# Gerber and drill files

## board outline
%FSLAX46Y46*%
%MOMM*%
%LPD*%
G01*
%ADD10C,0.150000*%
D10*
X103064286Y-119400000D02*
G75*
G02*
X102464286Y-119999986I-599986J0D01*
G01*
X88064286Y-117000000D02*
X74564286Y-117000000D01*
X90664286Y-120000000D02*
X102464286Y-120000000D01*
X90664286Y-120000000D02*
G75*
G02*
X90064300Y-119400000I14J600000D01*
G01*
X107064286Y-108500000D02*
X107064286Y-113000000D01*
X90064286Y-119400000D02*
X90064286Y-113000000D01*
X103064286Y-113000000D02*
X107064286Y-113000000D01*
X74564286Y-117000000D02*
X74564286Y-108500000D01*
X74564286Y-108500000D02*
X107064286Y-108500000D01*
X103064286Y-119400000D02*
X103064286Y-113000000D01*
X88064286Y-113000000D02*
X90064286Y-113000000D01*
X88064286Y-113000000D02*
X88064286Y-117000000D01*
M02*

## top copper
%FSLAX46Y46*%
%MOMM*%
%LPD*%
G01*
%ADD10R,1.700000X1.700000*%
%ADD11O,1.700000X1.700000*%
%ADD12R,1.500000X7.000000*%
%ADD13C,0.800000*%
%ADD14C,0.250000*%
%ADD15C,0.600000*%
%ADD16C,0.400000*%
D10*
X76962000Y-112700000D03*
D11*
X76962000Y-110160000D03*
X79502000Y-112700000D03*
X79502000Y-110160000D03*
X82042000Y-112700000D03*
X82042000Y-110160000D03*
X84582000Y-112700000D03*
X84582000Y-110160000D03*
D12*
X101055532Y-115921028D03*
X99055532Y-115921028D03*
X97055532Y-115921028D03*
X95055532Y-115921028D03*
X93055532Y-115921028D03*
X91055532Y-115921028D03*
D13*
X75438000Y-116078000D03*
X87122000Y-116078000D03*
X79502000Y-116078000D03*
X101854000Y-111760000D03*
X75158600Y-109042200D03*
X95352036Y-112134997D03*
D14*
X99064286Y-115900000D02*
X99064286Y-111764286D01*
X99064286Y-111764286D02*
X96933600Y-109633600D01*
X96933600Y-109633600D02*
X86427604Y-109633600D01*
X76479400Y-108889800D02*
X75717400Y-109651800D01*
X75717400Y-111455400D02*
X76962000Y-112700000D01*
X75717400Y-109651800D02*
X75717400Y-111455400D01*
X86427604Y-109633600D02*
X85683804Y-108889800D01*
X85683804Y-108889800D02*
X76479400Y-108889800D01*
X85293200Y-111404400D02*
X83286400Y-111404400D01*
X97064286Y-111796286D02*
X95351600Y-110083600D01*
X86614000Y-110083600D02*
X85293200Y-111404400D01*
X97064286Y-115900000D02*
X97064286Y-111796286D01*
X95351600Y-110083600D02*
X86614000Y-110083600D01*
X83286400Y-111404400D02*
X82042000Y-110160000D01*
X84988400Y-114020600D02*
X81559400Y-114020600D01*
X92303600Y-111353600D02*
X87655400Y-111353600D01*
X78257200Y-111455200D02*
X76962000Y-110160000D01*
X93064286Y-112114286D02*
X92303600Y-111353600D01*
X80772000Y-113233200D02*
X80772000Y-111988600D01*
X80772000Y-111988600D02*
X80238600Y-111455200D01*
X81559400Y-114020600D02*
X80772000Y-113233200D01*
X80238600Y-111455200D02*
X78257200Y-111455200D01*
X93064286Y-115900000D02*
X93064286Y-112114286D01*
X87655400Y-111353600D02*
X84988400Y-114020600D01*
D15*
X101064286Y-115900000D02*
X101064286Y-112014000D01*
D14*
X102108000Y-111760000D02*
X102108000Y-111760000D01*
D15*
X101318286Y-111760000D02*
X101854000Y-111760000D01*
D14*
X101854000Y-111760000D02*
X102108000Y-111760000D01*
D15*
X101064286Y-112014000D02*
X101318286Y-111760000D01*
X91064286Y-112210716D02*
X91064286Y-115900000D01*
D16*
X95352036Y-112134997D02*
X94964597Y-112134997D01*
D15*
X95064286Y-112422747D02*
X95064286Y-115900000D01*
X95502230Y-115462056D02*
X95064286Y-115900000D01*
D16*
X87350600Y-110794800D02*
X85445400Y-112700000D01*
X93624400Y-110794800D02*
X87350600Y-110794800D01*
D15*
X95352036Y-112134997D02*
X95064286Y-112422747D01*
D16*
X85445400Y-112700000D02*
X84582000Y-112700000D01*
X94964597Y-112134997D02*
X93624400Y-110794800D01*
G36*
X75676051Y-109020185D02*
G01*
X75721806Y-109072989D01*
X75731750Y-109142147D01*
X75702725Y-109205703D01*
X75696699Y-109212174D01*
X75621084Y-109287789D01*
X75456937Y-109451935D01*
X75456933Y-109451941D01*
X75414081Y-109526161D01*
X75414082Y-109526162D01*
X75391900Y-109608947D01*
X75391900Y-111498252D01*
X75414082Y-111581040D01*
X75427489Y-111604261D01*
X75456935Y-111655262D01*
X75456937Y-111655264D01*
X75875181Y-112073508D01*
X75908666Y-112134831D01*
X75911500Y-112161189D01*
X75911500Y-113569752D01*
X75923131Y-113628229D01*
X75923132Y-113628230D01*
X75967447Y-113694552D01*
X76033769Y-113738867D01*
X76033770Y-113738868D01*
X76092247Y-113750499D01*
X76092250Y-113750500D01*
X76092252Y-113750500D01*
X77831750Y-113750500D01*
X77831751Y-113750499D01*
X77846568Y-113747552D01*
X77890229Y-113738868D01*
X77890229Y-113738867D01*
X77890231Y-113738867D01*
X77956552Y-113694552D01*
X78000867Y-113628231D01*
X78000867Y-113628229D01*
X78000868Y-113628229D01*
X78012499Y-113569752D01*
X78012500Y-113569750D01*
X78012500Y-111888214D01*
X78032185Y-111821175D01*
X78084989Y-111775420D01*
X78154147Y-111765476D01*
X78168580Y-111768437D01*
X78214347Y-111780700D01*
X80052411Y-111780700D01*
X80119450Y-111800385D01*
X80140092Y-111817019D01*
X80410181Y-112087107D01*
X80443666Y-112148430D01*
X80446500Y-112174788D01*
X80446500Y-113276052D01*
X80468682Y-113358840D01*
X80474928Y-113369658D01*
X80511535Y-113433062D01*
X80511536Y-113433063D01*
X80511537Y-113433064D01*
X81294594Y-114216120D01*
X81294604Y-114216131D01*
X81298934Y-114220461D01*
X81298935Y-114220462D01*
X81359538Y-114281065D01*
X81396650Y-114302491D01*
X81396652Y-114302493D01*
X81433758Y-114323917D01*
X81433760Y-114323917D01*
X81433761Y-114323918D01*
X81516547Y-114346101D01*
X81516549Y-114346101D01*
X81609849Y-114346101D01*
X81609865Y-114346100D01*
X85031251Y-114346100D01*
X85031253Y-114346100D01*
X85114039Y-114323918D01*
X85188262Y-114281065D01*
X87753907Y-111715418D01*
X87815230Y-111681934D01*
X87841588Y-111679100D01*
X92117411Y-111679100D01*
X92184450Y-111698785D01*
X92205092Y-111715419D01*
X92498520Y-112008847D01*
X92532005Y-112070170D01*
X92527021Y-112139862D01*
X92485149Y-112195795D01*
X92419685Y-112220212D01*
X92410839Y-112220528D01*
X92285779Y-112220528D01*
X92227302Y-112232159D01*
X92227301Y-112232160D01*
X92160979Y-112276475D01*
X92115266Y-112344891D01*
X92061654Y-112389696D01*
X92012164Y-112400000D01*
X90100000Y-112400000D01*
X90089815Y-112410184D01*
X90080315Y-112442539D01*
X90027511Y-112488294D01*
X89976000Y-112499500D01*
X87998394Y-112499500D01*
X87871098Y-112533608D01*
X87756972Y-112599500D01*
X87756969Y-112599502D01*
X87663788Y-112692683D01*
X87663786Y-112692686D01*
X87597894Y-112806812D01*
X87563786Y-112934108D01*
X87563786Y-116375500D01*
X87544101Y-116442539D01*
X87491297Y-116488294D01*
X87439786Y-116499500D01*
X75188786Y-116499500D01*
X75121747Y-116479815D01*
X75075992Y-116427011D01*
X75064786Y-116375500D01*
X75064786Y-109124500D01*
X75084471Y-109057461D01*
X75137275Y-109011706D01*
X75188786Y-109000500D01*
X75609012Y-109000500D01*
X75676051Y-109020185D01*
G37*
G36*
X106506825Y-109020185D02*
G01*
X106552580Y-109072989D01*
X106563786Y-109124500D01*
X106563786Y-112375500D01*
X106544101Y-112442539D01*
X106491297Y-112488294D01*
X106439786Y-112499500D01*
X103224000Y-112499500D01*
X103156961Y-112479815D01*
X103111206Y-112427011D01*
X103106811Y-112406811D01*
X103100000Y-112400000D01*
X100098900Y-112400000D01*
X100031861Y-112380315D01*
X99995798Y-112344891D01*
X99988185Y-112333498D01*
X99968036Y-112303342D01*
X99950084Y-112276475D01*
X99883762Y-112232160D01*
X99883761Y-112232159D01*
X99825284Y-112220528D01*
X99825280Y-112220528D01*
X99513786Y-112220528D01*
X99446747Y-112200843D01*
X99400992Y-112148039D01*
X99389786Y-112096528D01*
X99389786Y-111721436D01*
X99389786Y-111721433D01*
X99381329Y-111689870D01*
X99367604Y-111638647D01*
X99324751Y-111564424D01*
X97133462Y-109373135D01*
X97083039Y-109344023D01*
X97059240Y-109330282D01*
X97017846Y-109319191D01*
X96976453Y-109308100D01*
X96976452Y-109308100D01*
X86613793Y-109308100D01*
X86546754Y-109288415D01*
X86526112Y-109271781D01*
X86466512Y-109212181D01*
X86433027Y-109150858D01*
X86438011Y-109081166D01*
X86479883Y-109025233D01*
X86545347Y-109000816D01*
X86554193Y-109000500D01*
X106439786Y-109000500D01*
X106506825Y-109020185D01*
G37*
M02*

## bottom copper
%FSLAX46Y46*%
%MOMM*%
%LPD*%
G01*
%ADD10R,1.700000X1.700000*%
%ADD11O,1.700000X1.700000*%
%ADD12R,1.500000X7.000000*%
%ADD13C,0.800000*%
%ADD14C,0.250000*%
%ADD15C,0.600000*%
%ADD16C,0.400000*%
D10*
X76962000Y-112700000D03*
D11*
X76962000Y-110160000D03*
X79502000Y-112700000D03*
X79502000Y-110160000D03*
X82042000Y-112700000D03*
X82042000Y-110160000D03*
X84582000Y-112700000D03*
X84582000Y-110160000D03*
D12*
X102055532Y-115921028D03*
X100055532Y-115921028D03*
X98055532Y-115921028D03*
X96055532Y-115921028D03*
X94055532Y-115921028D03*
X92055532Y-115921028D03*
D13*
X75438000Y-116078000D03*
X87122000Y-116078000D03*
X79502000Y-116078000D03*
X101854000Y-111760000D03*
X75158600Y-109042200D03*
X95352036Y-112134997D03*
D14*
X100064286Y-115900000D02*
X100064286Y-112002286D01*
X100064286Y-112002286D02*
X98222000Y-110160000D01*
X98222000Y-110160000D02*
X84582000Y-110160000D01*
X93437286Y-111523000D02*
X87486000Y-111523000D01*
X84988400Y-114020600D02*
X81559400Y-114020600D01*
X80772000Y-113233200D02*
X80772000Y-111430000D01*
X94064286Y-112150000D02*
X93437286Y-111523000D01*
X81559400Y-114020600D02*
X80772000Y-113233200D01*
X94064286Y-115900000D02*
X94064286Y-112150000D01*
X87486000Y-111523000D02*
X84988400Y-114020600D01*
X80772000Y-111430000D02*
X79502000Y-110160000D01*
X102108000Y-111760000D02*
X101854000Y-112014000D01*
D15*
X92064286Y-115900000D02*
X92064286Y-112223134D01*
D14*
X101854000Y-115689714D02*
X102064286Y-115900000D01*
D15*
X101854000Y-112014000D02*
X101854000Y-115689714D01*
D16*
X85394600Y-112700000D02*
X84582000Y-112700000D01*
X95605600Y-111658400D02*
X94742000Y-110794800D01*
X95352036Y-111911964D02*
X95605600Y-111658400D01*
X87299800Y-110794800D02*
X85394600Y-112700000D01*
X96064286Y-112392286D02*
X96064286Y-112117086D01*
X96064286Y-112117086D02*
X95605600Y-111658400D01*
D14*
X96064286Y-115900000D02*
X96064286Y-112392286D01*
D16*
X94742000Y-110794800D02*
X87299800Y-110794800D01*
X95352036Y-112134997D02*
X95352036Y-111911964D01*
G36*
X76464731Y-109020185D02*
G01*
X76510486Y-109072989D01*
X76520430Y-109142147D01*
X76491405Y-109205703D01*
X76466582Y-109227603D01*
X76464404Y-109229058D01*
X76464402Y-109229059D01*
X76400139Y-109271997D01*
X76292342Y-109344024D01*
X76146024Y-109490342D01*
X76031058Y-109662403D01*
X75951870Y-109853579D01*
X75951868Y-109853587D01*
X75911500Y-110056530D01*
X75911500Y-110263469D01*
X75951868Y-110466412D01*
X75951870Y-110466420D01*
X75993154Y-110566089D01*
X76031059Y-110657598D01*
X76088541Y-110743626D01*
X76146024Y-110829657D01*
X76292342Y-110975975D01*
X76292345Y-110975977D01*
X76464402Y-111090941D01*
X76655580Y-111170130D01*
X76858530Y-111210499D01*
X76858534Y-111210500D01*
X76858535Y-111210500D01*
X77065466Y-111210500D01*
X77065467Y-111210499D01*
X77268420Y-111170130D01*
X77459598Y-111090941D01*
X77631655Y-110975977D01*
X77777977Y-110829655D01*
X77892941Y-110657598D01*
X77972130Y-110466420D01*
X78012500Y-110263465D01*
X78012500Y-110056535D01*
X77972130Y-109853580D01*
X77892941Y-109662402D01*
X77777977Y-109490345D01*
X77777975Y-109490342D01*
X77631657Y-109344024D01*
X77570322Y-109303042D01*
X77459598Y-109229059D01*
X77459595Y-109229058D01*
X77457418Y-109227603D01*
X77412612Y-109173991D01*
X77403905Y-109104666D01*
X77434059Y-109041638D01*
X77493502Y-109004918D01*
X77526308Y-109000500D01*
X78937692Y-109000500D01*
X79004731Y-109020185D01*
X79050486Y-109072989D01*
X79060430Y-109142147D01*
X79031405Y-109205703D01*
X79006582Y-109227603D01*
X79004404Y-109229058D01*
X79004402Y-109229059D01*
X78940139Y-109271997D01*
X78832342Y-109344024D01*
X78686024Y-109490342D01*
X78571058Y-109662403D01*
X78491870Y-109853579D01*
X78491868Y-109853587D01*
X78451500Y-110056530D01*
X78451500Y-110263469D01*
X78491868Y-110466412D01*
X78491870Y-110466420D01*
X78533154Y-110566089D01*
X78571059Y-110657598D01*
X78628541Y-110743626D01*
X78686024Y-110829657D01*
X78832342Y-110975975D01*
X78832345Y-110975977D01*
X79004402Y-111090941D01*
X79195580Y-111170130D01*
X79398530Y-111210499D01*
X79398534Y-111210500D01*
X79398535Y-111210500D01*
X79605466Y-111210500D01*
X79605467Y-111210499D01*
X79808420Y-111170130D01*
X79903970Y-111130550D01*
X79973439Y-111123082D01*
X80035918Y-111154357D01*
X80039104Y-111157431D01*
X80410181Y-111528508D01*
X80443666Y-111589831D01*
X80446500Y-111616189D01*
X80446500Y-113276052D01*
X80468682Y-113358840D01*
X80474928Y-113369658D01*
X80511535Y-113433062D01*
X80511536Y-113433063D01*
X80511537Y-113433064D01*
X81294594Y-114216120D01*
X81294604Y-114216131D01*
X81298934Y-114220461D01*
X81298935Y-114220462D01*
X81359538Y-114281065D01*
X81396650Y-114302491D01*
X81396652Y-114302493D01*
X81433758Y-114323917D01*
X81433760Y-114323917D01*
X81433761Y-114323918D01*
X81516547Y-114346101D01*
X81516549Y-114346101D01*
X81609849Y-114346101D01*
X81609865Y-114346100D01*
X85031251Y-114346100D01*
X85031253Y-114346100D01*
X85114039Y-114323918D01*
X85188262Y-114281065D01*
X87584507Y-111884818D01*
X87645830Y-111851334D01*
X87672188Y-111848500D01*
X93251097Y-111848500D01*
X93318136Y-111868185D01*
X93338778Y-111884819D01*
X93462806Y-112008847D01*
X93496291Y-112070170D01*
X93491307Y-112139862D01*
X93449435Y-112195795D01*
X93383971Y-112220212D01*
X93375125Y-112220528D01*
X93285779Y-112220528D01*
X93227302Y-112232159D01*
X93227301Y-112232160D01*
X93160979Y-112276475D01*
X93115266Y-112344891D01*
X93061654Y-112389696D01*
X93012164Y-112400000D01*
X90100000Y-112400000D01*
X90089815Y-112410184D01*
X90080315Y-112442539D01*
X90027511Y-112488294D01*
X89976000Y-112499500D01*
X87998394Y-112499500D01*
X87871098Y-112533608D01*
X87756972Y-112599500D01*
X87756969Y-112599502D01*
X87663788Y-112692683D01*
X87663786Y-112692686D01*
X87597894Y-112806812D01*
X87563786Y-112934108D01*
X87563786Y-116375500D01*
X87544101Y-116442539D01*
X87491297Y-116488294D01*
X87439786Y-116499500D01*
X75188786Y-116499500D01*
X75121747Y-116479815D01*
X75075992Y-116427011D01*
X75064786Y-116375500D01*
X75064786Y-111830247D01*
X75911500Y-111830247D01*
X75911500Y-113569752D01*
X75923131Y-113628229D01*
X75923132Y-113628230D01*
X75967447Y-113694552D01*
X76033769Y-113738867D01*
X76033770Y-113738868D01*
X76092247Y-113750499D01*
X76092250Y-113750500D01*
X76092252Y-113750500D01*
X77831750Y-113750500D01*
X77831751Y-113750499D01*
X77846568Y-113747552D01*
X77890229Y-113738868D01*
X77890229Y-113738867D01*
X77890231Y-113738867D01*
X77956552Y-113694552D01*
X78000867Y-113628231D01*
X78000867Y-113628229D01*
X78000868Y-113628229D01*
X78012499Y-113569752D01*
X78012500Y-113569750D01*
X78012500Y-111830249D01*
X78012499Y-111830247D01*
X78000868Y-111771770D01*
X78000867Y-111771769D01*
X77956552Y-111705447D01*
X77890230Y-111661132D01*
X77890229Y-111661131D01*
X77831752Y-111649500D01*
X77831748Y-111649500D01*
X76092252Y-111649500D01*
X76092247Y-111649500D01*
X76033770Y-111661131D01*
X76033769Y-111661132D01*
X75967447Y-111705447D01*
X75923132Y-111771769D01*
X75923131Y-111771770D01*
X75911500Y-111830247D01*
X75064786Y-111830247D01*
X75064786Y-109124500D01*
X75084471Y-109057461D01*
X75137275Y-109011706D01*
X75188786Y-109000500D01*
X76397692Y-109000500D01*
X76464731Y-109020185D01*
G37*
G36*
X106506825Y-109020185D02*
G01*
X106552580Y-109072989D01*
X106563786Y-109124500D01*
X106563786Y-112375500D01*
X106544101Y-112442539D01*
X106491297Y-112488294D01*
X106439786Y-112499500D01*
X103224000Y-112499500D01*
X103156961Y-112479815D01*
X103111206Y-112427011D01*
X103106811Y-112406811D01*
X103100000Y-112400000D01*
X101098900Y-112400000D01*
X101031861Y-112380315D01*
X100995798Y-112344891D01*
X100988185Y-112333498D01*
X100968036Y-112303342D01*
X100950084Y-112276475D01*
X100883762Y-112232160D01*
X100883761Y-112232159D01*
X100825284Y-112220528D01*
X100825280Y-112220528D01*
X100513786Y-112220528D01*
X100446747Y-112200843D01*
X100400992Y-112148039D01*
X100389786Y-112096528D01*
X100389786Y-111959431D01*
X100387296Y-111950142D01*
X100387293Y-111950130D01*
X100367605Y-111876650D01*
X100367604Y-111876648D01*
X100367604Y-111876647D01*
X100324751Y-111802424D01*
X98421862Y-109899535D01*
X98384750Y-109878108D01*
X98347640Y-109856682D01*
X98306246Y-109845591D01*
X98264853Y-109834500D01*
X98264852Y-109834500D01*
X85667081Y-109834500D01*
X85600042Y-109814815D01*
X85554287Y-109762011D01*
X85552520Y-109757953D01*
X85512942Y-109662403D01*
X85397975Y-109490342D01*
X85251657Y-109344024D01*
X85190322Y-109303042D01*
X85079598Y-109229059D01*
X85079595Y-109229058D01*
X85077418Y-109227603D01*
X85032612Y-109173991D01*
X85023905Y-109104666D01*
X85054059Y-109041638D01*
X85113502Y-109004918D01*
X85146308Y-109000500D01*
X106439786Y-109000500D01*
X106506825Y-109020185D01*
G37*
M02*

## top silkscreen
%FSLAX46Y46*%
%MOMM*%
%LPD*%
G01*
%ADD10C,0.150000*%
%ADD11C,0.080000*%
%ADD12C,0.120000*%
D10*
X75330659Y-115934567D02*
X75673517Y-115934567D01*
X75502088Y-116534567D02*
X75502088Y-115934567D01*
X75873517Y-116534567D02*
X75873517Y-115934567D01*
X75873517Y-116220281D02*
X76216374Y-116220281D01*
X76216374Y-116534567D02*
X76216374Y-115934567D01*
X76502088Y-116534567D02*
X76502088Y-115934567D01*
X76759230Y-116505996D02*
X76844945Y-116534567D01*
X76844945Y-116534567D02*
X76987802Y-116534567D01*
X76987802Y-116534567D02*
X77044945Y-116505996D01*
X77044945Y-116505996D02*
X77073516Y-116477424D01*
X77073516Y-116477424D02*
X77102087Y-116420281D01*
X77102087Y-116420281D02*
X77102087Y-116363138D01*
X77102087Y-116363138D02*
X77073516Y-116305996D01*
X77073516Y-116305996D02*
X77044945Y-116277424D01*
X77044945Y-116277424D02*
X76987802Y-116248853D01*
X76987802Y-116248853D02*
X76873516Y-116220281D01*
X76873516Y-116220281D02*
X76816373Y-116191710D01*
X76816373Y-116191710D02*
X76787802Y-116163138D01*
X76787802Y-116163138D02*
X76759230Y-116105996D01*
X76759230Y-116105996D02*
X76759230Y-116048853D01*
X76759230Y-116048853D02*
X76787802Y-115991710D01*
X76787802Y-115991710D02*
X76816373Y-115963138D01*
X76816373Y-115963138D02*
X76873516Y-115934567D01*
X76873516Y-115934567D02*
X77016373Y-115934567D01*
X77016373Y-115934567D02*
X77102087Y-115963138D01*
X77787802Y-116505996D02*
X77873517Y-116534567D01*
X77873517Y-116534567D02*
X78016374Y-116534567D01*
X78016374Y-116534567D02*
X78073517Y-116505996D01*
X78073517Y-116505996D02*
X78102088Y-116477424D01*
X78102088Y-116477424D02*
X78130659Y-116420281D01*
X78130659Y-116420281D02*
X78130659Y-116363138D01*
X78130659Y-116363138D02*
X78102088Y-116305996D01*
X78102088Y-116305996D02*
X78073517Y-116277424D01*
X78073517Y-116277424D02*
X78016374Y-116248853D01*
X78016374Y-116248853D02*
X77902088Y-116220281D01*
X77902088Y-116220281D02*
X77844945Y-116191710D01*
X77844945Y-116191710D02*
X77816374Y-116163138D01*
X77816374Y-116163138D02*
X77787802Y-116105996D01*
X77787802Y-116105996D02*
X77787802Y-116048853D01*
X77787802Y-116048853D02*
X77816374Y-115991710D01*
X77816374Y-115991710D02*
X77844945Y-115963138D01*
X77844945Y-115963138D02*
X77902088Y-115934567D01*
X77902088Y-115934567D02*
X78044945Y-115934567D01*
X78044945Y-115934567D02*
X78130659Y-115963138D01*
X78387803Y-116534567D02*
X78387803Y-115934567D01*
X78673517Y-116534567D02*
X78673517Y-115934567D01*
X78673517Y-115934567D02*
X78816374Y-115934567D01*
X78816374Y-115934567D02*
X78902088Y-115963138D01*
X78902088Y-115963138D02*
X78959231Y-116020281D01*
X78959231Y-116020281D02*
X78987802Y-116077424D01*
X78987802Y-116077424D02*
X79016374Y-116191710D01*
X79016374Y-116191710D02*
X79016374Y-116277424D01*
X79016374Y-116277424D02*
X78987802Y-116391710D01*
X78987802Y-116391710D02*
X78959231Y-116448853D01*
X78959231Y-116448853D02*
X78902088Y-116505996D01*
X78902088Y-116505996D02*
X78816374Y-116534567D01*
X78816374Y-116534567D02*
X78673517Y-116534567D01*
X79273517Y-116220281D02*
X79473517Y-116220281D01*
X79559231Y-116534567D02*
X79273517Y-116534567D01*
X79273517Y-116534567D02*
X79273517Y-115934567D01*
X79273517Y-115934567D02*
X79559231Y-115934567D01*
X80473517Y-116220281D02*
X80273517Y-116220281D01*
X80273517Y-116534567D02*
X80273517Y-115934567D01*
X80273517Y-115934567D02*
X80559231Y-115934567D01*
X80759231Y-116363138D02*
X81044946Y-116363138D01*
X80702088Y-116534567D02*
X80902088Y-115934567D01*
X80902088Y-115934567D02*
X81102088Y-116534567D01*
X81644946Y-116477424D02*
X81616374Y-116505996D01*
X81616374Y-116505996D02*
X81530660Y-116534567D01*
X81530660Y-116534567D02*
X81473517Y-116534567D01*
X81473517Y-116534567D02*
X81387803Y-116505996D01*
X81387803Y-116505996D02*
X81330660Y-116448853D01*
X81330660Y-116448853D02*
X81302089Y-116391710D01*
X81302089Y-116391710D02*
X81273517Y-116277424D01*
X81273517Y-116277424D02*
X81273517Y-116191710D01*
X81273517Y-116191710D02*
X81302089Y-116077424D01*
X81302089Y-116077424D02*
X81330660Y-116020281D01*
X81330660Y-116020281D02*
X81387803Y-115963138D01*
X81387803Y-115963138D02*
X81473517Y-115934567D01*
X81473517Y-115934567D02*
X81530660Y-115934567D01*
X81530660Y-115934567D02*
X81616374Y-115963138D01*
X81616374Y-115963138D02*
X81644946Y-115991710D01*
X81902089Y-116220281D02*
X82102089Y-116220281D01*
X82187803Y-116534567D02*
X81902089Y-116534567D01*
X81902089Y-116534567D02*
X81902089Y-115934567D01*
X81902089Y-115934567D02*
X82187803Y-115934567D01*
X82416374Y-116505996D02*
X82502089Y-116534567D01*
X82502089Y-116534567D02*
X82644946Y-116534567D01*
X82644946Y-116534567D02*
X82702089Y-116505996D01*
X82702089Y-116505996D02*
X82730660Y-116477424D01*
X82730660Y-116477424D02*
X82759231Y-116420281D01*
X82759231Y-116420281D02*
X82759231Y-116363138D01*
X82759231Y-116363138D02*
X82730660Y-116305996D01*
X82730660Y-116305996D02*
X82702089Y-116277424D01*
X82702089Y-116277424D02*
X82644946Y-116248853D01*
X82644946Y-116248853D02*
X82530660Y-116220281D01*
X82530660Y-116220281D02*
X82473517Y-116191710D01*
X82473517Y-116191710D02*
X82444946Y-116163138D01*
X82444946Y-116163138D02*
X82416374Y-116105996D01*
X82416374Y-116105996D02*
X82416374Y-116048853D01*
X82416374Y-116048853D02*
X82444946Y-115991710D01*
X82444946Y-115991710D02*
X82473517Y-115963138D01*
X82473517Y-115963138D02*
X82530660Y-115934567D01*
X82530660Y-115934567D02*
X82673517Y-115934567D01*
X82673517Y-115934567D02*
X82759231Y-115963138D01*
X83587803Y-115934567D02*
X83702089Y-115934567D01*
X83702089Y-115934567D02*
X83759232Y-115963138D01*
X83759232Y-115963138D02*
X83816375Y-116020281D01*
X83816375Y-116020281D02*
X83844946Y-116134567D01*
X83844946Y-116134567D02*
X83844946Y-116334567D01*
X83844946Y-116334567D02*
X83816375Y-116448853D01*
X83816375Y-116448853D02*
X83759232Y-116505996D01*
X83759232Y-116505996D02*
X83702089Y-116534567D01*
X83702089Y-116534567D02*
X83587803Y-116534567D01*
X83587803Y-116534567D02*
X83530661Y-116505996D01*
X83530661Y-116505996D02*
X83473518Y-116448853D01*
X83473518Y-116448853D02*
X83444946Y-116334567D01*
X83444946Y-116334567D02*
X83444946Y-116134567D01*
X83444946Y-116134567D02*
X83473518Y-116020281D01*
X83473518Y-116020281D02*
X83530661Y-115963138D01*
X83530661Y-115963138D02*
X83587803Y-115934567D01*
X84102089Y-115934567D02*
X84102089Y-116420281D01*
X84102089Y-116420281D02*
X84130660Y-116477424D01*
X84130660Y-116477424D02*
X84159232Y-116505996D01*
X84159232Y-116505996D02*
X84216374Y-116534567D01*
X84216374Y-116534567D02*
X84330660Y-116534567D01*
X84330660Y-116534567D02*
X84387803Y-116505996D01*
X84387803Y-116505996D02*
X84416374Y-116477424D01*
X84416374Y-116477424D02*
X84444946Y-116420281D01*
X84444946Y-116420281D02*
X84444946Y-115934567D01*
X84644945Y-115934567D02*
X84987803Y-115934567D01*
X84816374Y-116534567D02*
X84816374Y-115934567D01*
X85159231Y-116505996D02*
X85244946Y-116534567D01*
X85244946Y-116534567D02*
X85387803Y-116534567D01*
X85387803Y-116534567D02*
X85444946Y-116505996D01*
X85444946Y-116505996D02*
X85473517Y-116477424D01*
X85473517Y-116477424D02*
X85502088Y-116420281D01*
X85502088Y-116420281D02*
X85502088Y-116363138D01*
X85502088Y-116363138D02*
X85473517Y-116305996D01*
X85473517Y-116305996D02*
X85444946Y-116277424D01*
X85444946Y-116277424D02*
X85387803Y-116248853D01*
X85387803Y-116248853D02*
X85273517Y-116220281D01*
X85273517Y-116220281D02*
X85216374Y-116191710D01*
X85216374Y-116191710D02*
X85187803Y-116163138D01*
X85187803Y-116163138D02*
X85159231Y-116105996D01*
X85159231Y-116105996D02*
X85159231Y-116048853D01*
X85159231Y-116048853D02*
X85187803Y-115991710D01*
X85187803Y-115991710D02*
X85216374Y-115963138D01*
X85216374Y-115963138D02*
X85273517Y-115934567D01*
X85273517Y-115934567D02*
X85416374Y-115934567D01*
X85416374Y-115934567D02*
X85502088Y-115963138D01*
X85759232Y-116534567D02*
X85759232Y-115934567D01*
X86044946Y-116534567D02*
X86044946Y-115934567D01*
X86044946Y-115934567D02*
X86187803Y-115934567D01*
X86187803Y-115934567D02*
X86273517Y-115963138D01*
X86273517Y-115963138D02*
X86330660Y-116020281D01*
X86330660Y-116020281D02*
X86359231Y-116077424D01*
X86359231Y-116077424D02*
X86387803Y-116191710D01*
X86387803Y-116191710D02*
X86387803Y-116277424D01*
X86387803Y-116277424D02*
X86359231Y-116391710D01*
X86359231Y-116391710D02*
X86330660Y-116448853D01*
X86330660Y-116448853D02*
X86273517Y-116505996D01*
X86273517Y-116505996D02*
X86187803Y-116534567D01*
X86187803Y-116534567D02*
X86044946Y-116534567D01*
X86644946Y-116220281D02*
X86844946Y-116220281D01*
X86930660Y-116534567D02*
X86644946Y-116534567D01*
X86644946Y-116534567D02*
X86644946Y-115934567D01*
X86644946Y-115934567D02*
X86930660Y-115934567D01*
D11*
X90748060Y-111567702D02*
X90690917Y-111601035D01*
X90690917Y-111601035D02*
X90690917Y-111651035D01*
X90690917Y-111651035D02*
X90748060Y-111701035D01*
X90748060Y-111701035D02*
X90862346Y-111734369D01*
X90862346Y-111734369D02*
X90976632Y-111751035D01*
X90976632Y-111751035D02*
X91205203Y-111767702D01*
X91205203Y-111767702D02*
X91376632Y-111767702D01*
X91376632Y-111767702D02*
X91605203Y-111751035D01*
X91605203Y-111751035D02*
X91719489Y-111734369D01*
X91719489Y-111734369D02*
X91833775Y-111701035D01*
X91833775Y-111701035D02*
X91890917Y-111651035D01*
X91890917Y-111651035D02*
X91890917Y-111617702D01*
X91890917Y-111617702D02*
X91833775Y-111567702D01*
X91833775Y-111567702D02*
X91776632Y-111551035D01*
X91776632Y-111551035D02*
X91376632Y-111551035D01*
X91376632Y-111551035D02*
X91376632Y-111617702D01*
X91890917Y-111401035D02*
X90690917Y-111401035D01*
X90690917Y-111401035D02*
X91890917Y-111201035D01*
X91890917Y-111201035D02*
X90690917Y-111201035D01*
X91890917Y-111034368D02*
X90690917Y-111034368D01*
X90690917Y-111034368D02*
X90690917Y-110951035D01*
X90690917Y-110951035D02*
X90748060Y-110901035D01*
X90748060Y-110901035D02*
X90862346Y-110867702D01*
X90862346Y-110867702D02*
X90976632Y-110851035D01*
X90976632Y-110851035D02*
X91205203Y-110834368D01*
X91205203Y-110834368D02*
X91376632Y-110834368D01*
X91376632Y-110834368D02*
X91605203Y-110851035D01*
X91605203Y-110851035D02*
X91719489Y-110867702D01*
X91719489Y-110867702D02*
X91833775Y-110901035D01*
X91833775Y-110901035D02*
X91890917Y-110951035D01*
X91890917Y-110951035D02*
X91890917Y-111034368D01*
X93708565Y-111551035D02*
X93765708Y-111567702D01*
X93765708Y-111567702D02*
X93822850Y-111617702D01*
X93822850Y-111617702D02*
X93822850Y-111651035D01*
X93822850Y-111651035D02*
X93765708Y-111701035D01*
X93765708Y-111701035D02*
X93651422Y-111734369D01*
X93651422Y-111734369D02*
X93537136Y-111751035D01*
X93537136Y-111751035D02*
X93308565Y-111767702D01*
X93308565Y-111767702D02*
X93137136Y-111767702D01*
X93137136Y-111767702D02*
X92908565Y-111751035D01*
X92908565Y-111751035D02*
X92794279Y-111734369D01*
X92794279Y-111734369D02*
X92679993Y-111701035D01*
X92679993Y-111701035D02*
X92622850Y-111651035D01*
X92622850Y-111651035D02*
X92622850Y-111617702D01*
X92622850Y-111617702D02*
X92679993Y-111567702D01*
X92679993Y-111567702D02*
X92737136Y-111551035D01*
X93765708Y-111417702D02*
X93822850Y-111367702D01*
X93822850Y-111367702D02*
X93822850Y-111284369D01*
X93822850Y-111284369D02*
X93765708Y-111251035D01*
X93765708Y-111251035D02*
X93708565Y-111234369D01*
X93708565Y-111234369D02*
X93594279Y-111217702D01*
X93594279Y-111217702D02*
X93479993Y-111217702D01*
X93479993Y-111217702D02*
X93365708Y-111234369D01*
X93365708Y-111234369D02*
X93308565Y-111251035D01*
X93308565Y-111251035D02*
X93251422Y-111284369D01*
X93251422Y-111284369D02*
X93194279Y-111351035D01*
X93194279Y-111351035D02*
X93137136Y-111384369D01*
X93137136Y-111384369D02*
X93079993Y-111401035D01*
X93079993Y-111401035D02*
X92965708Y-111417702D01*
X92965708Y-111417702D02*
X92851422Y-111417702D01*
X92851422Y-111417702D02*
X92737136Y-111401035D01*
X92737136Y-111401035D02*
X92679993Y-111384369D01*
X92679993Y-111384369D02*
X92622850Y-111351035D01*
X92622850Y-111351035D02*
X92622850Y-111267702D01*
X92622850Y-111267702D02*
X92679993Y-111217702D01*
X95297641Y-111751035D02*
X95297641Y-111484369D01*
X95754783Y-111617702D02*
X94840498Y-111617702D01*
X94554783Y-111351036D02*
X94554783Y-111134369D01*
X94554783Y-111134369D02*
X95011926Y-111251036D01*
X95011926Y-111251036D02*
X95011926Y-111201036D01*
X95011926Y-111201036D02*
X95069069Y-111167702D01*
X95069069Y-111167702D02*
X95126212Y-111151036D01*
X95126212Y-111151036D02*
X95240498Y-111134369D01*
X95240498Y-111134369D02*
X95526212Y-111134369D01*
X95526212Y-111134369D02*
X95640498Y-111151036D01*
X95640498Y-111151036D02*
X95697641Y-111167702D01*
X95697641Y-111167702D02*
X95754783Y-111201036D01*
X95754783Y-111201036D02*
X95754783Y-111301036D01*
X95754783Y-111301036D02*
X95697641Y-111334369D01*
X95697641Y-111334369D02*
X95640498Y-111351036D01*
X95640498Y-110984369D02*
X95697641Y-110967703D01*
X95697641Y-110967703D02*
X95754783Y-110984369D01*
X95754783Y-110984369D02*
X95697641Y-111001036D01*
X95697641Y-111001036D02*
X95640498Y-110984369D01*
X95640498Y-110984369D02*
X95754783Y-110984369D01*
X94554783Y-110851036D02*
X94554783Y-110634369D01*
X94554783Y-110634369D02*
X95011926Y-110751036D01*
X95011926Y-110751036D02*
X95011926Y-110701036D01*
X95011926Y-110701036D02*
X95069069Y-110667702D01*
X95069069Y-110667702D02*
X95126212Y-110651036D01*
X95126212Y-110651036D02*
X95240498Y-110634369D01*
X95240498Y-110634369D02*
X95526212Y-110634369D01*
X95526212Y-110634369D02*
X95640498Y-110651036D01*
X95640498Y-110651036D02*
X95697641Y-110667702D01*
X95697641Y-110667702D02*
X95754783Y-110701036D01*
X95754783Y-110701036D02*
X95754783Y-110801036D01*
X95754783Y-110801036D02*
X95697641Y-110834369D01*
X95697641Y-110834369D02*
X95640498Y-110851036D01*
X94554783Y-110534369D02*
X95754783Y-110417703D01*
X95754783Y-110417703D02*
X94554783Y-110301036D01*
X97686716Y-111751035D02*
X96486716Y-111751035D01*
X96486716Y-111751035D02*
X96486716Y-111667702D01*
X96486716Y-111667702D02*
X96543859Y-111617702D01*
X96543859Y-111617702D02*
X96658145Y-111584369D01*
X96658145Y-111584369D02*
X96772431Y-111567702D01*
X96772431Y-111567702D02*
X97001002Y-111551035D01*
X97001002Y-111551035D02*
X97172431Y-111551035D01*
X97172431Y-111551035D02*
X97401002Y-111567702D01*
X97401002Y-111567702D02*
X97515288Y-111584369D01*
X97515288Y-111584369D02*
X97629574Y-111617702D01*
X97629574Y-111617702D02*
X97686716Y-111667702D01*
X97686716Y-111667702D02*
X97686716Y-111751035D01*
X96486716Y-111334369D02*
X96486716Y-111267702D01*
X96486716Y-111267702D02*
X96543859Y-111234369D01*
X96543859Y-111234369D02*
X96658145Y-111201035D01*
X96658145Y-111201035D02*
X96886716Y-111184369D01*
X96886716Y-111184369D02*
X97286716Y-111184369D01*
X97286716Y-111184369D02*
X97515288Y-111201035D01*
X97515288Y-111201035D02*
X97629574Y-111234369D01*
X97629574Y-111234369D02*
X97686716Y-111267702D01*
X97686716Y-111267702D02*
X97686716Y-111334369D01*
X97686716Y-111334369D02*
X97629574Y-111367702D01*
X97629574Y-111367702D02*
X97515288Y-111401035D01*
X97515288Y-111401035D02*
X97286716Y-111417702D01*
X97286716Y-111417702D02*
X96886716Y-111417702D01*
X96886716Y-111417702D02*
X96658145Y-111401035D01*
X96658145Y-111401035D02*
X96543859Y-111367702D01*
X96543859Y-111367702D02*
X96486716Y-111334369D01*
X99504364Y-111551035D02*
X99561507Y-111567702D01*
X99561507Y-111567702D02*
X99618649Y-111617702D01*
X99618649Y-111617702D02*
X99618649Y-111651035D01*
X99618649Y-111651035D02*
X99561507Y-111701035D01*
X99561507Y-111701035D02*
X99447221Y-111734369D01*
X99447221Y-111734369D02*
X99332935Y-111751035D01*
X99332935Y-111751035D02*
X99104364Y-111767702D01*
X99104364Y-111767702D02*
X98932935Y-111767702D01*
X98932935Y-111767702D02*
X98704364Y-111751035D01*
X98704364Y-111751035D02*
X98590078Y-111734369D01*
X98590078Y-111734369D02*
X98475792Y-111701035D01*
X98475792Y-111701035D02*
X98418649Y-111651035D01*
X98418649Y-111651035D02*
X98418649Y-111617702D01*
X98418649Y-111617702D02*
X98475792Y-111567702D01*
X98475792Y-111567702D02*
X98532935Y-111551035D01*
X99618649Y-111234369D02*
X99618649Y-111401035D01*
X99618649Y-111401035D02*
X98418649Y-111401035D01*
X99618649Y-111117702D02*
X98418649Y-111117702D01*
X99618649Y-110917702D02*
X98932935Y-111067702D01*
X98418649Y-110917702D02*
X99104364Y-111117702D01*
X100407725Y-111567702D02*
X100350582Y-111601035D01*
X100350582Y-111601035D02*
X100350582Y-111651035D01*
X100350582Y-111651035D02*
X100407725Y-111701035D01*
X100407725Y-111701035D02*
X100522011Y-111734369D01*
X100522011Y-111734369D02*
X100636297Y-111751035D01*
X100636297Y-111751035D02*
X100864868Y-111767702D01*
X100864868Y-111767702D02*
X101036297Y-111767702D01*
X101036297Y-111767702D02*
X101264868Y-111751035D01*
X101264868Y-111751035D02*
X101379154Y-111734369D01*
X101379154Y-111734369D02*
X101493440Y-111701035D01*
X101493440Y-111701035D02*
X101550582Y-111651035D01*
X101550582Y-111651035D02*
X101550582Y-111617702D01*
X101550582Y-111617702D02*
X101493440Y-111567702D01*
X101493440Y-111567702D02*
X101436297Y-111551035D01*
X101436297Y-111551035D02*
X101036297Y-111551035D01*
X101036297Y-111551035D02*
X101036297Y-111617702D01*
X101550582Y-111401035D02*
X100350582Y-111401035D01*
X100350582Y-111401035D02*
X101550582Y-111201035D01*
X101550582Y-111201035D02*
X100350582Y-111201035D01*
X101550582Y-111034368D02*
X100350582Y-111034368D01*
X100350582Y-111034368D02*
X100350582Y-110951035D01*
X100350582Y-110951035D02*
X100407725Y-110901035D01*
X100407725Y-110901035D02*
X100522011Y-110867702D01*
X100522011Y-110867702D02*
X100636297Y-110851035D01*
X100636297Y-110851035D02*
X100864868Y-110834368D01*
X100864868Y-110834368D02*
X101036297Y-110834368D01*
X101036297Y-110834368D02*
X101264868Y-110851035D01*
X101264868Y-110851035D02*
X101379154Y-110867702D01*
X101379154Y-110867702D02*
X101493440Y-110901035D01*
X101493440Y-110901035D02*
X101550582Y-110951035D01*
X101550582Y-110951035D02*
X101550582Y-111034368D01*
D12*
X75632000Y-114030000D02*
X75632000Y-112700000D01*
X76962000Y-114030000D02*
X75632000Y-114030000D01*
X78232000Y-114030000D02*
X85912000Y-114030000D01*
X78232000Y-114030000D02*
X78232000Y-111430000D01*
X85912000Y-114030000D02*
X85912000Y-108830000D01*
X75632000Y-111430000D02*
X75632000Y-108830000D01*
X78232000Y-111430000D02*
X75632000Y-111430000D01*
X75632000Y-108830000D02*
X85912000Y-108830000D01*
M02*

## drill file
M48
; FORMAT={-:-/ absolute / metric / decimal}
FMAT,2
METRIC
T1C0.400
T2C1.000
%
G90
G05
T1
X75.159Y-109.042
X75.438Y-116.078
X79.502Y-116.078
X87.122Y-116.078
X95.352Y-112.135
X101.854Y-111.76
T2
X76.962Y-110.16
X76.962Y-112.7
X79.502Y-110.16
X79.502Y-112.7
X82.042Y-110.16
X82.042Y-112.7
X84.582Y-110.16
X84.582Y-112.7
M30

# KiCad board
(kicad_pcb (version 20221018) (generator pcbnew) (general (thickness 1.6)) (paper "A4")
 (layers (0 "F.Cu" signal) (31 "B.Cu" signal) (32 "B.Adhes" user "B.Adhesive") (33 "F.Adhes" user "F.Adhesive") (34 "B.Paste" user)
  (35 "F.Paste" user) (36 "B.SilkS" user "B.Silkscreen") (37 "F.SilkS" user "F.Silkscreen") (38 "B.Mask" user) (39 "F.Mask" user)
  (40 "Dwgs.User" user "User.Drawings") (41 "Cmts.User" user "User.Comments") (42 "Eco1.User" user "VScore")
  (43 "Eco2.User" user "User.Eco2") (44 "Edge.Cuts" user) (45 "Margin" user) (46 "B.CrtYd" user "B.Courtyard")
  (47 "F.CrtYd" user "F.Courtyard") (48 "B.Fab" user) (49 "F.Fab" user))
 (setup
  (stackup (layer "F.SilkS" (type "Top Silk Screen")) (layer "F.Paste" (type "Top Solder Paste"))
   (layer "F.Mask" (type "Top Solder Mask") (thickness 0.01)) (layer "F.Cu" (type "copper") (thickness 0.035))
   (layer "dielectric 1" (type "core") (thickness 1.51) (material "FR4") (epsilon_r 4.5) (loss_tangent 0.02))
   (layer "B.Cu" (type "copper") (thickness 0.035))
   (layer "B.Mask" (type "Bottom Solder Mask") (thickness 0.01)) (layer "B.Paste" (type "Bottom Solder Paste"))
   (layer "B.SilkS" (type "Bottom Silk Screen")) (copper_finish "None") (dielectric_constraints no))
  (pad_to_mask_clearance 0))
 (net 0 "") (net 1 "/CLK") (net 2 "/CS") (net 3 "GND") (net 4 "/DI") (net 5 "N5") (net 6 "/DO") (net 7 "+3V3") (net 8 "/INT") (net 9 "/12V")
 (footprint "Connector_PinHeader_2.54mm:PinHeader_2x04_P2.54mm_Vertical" (layer "F.Cu") (at 76.962 112.7 90)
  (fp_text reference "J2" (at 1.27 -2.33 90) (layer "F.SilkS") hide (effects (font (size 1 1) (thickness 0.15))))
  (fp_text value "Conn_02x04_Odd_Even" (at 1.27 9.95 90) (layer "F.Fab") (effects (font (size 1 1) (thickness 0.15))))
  (fp_line (start -1.33 -1.33) (end 0 -1.33) (stroke (width 0.12) (type solid)) (layer "F.SilkS"))
  (fp_line (start -1.33 0) (end -1.33 -1.33) (stroke (width 0.12) (type solid)) (layer "F.SilkS"))
  (fp_line (start -1.33 1.27) (end -1.33 8.95) (stroke (width 0.12) (type solid)) (layer "F.SilkS"))
  (fp_line (start -1.33 1.27) (end 1.27 1.27) (stroke (width 0.12) (type solid)) (layer "F.SilkS"))
  (fp_line (start -1.33 8.95) (end 3.87 8.95) (stroke (width 0.12) (type solid)) (layer "F.SilkS"))
  (fp_line (start 1.27 -1.33) (end 3.87 -1.33) (stroke (width 0.12) (type solid)) (layer "F.SilkS"))
  (fp_line (start 1.27 1.27) (end 1.27 -1.33) (stroke (width 0.12) (type solid)) (layer "F.SilkS"))
  (fp_line (start 3.87 -1.33) (end 3.87 8.95) (stroke (width 0.12) (type solid)) (layer "F.SilkS"))
  (pad "1" thru_hole rect (at 0 0 90) (size 1.7 1.7) (drill 1) (layers "*.Cu" "*.Mask") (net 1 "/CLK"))
  (pad "2" thru_hole oval (at 2.54 0 90) (size 1.7 1.7) (drill 1) (layers "*.Cu" "*.Mask") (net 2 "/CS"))
  (pad "3" thru_hole oval (at 0 2.54 90) (size 1.7 1.7) (drill 1) (layers "*.Cu" "*.Mask") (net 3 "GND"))
  (pad "4" thru_hole oval (at 2.54 2.54 90) (size 1.7 1.7) (drill 1) (layers "*.Cu" "*.Mask") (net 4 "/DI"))
  (pad "5" thru_hole oval (at 0 5.08 90) (size 1.7 1.7) (drill 1) (layers "*.Cu" "*.Mask") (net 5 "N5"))
  (pad "6" thru_hole oval (at 2.54 5.08 90) (size 1.7 1.7) (drill 1) (layers "*.Cu" "*.Mask") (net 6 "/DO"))
  (pad "7" thru_hole oval (at 0 7.62 90) (size 1.7 1.7) (drill 1) (layers "*.Cu" "*.Mask") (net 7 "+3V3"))
  (pad "8" thru_hole oval (at 2.54 7.62 90) (size 1.7 1.7) (drill 1) (layers "*.Cu" "*.Mask") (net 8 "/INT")))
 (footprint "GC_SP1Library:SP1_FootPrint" (layer "B.Cu") (at 102.055532 115.921028 180)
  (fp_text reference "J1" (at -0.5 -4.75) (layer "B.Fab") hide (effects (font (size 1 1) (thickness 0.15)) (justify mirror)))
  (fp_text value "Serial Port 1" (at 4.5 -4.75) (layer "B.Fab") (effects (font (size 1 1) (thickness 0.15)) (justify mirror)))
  (pad "1" smd rect (at 0 0 180) (size 1.5 7) (layers "B.Cu" "B.Mask") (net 3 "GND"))
  (pad "2" smd rect (at 1 0 180) (size 1.5 7) (layers "F.Cu" "F.Mask") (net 3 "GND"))
  (pad "3" smd rect (at 2 0 180) (size 1.5 7) (layers "B.Cu" "B.Mask") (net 8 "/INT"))
  (pad "4" smd rect (at 3 0 180) (size 1.5 7) (layers "F.Cu" "F.Mask") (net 1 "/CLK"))
  (pad "5" smd rect (at 4 0 180) (size 1.5 7) (layers "B.Cu" "B.Mask") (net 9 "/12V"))
  (pad "6" smd rect (at 5 0 180) (size 1.5 7) (layers "F.Cu" "F.Mask") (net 6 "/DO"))
  (pad "7" smd rect (at 6 0 180) (size 1.5 7) (layers "B.Cu" "B.Mask") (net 7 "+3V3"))
  (pad "8" smd rect (at 7 0 180) (size 1.5 7) (layers "F.Cu" "F.Mask") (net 7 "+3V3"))
  (pad "9" smd rect (at 8 0 180) (size 1.5 7) (layers "B.Cu" "B.Mask") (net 4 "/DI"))
  (pad "10" smd rect (at 9 0 180) (size 1.5 7) (layers "F.Cu" "F.Mask") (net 2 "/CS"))
  (pad "11" smd rect (at 10 0 180) (size 1.5 7) (layers "B.Cu" "B.Mask") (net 3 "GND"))
  (pad "12" smd rect (at 11 0 180) (size 1.5 7) (layers "F.Cu" "F.Mask") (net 3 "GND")))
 (gr_arc (start 103.064286 119.4) (mid 102.888549 119.824259) (end 102.464286 120) (stroke (width 0.15) (type solid)) (layer "Edge.Cuts"))
 (gr_line (start 88.064286 117) (end 74.564286 117) (stroke (width 0.15) (type solid)) (layer "Edge.Cuts"))
 (gr_line (start 90.664286 120) (end 102.464286 120) (stroke (width 0.15) (type solid)) (layer "Edge.Cuts"))
 (gr_arc (start 90.664286 120) (mid 90.240022 119.824264) (end 90.064286 119.4) (stroke (width 0.15) (type solid)) (layer "Edge.Cuts"))
 (gr_line (start 107.064286 108.5) (end 107.064286 113) (stroke (width 0.15) (type default)) (layer "Edge.Cuts"))
 (gr_line (start 90.064286 119.4) (end 90.064286 113) (stroke (width 0.15) (type solid)) (layer "Edge.Cuts"))
 (gr_line (start 103.064286 113) (end 107.064286 113) (stroke (width 0.15) (type solid)) (layer "Edge.Cuts"))
 (gr_line (start 74.564286 117) (end 74.564286 108.5) (stroke (width 0.15) (type solid)) (layer "Edge.Cuts"))
 (gr_line (start 74.564286 108.5) (end 107.064286 108.5) (stroke (width 0.15) (type solid)) (layer "Edge.Cuts"))
 (gr_line (start 103.064286 119.4) (end 103.064286 113) (stroke (width 0.15) (type solid)) (layer "Edge.Cuts"))
 (gr_line (start 88.064286 113) (end 90.064286 113) (stroke (width 0.15) (type solid)) (layer "Edge.Cuts"))
 (gr_line (start 88.064286 113) (end 88.064286 117) (stroke (width 0.15) (type solid)) (layer "Edge.Cuts"))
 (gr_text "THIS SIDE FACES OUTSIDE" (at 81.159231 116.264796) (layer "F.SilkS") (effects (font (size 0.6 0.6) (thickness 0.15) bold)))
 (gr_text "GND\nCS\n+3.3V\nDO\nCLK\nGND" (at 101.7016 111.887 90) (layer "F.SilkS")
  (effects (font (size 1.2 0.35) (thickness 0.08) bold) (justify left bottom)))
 (segment (start 100.064286 115.9) (end 100.064286 112.002286) (width 0.25) (layer "B.Cu") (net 8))
 (segment (start 100.064286 112.002286) (end 98.222 110.16) (width 0.25) (layer "B.Cu") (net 8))
 (segment (start 98.222 110.16) (end 84.582 110.16) (width 0.25) (layer "B.Cu") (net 8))
 (segment (start 93.437286 111.523) (end 87.486 111.523) (width 0.25) (layer "B.Cu") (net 4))
 (segment (start 84.9884 114.0206) (end 81.5594 114.0206) (width 0.25) (layer "B.Cu") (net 4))
 (segment (start 80.772 113.2332) (end 80.772 111.43) (width 0.25) (layer "B.Cu") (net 4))
 (segment (start 94.064286 112.15) (end 93.437286 111.523) (width 0.25) (layer "B.Cu") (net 4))
 (segment (start 81.5594 114.0206) (end 80.772 113.2332) (width 0.25) (layer "B.Cu") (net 4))
 (segment (start 94.064286 115.9) (end 94.064286 112.15) (width 0.25) (layer "B.Cu") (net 4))
 (segment (start 87.486 111.523) (end 84.9884 114.0206) (width 0.25) (layer "B.Cu") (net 4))
 (segment (start 80.772 111.43) (end 79.502 110.16) (width 0.25) (layer "B.Cu") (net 4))
 (segment (start 99.064286 115.9) (end 99.064286 111.764286) (width 0.25) (layer "F.Cu") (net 1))
 (segment (start 99.064286 111.764286) (end 96.9336 109.6336) (width 0.25) (layer "F.Cu") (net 1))
 (segment (start 96.9336 109.6336) (end 86.427604 109.6336) (width 0.25) (layer "F.Cu") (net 1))
 (segment (start 76.4794 108.8898) (end 75.7174 109.6518) (width 0.25) (layer "F.Cu") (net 1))
 (segment (start 75.7174 111.4554) (end 76.962 112.7) (width 0.25) (layer "F.Cu") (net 1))
 (segment (start 75.7174 109.6518) (end 75.7174 111.4554) (width 0.25) (layer "F.Cu") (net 1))
 (segment (start 86.427604 109.6336) (end 85.683804 108.8898) (width 0.25) (layer "F.Cu") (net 1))
 (segment (start 85.683804 108.8898) (end 76.4794 108.8898) (width 0.25) (layer "F.Cu") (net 1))
 (segment (start 85.2932 111.4044) (end 83.2864 111.4044) (width 0.25) (layer "F.Cu") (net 6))
 (segment (start 97.064286 111.796286) (end 95.3516 110.0836) (width 0.25) (layer "F.Cu") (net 6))
 (segment (start 86.614 110.0836) (end 85.2932 111.4044) (width 0.25) (layer "F.Cu") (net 6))
 (segment (start 97.064286 115.9) (end 97.064286 111.796286) (width 0.25) (layer "F.Cu") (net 6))
 (segment (start 95.3516 110.0836) (end 86.614 110.0836) (width 0.25) (layer "F.Cu") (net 6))
 (segment (start 83.2864 111.4044) (end 82.042 110.16) (width 0.25) (layer "F.Cu") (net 6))
 (segment (start 84.9884 114.0206) (end 81.5594 114.0206) (width 0.25) (layer "F.Cu") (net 2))
 (segment (start 92.3036 111.3536) (end 87.6554 111.3536) (width 0.25) (layer "F.Cu") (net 2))
 (segment (start 78.2572 111.4552) (end 76.962 110.16) (width 0.25) (layer "F.Cu") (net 2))
 (segment (start 93.064286 112.114286) (end 92.3036 111.3536) (width 0.25) (layer "F.Cu") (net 2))
 (segment (start 80.772 113.2332) (end 80.772 111.9886) (width 0.25) (layer "F.Cu") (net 2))
 (segment (start 80.772 111.9886) (end 80.2386 111.4552) (width 0.25) (layer "F.Cu") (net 2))
 (segment (start 81.5594 114.0206) (end 80.772 113.2332) (width 0.25) (layer "F.Cu") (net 2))
 (segment (start 80.2386 111.4552) (end 78.2572 111.4552) (width 0.25) (layer "F.Cu") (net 2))
 (segment (start 93.064286 115.9) (end 93.064286 112.114286) (width 0.25) (layer "F.Cu") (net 2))
 (segment (start 87.6554 111.3536) (end 84.9884 114.0206) (width 0.25) (layer "F.Cu") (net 2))
 (segment (start 101.064286 115.9) (end 101.064286 112.014) (width 0.6) (layer "F.Cu") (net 3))
 (segment (start 102.108 111.76) (end 102.108 111.76) (width 0.25) (layer "F.Cu") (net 3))
 (segment (start 101.318286 111.76) (end 101.854 111.76) (width 0.6) (layer "F.Cu") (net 3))
 (segment (start 101.854 111.76) (end 102.108 111.76) (width 0.25) (layer "F.Cu") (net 3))
 (segment (start 101.064286 112.014) (end 101.318286 111.76) (width 0.6) (layer "F.Cu") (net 3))
 (segment (start 91.064286 112.210716) (end 91.064286 115.9) (width 0.6) (layer "F.Cu") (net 3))
 (via (at 75.438 116.078) (size 0.8) (drill 0.4) (layers "F.Cu" "B.Cu") (free) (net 3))
 (via (at 87.122 116.078) (size 0.8) (drill 0.4) (layers "F.Cu" "B.Cu") (free) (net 3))
 (via (at 79.502 116.078) (size 0.8) (drill 0.4) (layers "F.Cu" "B.Cu") (free) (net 3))
 (via (at 101.854 111.76) (size 0.8) (drill 0.4) (layers "F.Cu" "B.Cu") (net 3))
 (via (at 75.1586 109.0422) (size 0.8) (drill 0.4) (layers "F.Cu" "B.Cu") (free) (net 3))
 (segment (start 102.108 111.76) (end 101.854 112.014) (width 0.25) (layer "B.Cu") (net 3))
 (segment (start 92.064286 115.9) (end 92.064286 112.223134) (width 0.6) (layer "B.Cu") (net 3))
 (segment (start 101.854 115.689714) (end 102.064286 115.9) (width 0.25) (layer "B.Cu") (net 3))
 (segment (start 101.854 112.014) (end 101.854 115.689714) (width 0.6) (layer "B.Cu") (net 3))
 (segment (start 95.352036 112.134997) (end 94.964597 112.134997) (width 0.4) (layer "F.Cu") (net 7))
 (segment (start 95.064286 112.422747) (end 95.064286 115.9) (width 0.6) (layer "F.Cu") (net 7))
 (segment (start 95.50223 115.462056) (end 95.064286 115.9) (width 0.6) (layer "F.Cu") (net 7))
 (segment (start 87.3506 110.7948) (end 85.4454 112.7) (width 0.4) (layer "F.Cu") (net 7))
 (segment (start 93.6244 110.7948) (end 87.3506 110.7948) (width 0.4) (layer "F.Cu") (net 7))
 (segment (start 95.352036 112.134997) (end 95.064286 112.422747) (width 0.6) (layer "F.Cu") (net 7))
 (segment (start 85.4454 112.7) (end 84.582 112.7) (width 0.4) (layer "F.Cu") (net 7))
 (segment (start 94.964597 112.134997) (end 93.6244 110.7948) (width 0.4) (layer "F.Cu") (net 7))
 (via (at 95.352036 112.134997) (size 0.8) (drill 0.4) (layers "F.Cu" "B.Cu") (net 7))
 (segment (start 85.3946 112.7) (end 84.582 112.7) (width 0.4) (layer "B.Cu") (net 7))
 (segment (start 95.6056 111.6584) (end 94.742 110.7948) (width 0.4) (layer "B.Cu") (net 7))
 (segment (start 95.352036 111.911964) (end 95.6056 111.6584) (width 0.4) (layer "B.Cu") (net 7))
 (segment (start 87.2998 110.7948) (end 85.3946 112.7) (width 0.4) (layer "B.Cu") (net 7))
 (segment (start 96.064286 112.392286) (end 96.064286 112.117086) (width 0.4) (layer "B.Cu") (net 7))
 (segment (start 96.064286 112.117086) (end 95.6056 111.6584) (width 0.4) (layer "B.Cu") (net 7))
 (segment (start 96.064286 115.9) (end 96.064286 112.392286) (width 0.25) (layer "B.Cu") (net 7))
 (segment (start 94.742 110.7948) (end 87.2998 110.7948) (width 0.4) (layer "B.Cu") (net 7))
 (segment (start 95.352036 112.134997) (end 95.352036 111.911964) (width 0.4) (layer "B.Cu") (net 7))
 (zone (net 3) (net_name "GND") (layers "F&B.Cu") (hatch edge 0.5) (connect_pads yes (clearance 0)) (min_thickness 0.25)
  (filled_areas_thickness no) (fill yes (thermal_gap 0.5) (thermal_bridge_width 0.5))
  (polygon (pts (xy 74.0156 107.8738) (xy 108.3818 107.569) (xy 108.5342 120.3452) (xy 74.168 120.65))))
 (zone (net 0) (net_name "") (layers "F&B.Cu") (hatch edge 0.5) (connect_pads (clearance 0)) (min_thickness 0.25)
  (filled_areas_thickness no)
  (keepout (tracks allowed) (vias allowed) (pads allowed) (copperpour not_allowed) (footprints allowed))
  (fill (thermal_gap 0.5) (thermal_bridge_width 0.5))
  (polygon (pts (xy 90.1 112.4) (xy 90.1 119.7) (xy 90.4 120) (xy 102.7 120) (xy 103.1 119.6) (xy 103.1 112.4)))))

